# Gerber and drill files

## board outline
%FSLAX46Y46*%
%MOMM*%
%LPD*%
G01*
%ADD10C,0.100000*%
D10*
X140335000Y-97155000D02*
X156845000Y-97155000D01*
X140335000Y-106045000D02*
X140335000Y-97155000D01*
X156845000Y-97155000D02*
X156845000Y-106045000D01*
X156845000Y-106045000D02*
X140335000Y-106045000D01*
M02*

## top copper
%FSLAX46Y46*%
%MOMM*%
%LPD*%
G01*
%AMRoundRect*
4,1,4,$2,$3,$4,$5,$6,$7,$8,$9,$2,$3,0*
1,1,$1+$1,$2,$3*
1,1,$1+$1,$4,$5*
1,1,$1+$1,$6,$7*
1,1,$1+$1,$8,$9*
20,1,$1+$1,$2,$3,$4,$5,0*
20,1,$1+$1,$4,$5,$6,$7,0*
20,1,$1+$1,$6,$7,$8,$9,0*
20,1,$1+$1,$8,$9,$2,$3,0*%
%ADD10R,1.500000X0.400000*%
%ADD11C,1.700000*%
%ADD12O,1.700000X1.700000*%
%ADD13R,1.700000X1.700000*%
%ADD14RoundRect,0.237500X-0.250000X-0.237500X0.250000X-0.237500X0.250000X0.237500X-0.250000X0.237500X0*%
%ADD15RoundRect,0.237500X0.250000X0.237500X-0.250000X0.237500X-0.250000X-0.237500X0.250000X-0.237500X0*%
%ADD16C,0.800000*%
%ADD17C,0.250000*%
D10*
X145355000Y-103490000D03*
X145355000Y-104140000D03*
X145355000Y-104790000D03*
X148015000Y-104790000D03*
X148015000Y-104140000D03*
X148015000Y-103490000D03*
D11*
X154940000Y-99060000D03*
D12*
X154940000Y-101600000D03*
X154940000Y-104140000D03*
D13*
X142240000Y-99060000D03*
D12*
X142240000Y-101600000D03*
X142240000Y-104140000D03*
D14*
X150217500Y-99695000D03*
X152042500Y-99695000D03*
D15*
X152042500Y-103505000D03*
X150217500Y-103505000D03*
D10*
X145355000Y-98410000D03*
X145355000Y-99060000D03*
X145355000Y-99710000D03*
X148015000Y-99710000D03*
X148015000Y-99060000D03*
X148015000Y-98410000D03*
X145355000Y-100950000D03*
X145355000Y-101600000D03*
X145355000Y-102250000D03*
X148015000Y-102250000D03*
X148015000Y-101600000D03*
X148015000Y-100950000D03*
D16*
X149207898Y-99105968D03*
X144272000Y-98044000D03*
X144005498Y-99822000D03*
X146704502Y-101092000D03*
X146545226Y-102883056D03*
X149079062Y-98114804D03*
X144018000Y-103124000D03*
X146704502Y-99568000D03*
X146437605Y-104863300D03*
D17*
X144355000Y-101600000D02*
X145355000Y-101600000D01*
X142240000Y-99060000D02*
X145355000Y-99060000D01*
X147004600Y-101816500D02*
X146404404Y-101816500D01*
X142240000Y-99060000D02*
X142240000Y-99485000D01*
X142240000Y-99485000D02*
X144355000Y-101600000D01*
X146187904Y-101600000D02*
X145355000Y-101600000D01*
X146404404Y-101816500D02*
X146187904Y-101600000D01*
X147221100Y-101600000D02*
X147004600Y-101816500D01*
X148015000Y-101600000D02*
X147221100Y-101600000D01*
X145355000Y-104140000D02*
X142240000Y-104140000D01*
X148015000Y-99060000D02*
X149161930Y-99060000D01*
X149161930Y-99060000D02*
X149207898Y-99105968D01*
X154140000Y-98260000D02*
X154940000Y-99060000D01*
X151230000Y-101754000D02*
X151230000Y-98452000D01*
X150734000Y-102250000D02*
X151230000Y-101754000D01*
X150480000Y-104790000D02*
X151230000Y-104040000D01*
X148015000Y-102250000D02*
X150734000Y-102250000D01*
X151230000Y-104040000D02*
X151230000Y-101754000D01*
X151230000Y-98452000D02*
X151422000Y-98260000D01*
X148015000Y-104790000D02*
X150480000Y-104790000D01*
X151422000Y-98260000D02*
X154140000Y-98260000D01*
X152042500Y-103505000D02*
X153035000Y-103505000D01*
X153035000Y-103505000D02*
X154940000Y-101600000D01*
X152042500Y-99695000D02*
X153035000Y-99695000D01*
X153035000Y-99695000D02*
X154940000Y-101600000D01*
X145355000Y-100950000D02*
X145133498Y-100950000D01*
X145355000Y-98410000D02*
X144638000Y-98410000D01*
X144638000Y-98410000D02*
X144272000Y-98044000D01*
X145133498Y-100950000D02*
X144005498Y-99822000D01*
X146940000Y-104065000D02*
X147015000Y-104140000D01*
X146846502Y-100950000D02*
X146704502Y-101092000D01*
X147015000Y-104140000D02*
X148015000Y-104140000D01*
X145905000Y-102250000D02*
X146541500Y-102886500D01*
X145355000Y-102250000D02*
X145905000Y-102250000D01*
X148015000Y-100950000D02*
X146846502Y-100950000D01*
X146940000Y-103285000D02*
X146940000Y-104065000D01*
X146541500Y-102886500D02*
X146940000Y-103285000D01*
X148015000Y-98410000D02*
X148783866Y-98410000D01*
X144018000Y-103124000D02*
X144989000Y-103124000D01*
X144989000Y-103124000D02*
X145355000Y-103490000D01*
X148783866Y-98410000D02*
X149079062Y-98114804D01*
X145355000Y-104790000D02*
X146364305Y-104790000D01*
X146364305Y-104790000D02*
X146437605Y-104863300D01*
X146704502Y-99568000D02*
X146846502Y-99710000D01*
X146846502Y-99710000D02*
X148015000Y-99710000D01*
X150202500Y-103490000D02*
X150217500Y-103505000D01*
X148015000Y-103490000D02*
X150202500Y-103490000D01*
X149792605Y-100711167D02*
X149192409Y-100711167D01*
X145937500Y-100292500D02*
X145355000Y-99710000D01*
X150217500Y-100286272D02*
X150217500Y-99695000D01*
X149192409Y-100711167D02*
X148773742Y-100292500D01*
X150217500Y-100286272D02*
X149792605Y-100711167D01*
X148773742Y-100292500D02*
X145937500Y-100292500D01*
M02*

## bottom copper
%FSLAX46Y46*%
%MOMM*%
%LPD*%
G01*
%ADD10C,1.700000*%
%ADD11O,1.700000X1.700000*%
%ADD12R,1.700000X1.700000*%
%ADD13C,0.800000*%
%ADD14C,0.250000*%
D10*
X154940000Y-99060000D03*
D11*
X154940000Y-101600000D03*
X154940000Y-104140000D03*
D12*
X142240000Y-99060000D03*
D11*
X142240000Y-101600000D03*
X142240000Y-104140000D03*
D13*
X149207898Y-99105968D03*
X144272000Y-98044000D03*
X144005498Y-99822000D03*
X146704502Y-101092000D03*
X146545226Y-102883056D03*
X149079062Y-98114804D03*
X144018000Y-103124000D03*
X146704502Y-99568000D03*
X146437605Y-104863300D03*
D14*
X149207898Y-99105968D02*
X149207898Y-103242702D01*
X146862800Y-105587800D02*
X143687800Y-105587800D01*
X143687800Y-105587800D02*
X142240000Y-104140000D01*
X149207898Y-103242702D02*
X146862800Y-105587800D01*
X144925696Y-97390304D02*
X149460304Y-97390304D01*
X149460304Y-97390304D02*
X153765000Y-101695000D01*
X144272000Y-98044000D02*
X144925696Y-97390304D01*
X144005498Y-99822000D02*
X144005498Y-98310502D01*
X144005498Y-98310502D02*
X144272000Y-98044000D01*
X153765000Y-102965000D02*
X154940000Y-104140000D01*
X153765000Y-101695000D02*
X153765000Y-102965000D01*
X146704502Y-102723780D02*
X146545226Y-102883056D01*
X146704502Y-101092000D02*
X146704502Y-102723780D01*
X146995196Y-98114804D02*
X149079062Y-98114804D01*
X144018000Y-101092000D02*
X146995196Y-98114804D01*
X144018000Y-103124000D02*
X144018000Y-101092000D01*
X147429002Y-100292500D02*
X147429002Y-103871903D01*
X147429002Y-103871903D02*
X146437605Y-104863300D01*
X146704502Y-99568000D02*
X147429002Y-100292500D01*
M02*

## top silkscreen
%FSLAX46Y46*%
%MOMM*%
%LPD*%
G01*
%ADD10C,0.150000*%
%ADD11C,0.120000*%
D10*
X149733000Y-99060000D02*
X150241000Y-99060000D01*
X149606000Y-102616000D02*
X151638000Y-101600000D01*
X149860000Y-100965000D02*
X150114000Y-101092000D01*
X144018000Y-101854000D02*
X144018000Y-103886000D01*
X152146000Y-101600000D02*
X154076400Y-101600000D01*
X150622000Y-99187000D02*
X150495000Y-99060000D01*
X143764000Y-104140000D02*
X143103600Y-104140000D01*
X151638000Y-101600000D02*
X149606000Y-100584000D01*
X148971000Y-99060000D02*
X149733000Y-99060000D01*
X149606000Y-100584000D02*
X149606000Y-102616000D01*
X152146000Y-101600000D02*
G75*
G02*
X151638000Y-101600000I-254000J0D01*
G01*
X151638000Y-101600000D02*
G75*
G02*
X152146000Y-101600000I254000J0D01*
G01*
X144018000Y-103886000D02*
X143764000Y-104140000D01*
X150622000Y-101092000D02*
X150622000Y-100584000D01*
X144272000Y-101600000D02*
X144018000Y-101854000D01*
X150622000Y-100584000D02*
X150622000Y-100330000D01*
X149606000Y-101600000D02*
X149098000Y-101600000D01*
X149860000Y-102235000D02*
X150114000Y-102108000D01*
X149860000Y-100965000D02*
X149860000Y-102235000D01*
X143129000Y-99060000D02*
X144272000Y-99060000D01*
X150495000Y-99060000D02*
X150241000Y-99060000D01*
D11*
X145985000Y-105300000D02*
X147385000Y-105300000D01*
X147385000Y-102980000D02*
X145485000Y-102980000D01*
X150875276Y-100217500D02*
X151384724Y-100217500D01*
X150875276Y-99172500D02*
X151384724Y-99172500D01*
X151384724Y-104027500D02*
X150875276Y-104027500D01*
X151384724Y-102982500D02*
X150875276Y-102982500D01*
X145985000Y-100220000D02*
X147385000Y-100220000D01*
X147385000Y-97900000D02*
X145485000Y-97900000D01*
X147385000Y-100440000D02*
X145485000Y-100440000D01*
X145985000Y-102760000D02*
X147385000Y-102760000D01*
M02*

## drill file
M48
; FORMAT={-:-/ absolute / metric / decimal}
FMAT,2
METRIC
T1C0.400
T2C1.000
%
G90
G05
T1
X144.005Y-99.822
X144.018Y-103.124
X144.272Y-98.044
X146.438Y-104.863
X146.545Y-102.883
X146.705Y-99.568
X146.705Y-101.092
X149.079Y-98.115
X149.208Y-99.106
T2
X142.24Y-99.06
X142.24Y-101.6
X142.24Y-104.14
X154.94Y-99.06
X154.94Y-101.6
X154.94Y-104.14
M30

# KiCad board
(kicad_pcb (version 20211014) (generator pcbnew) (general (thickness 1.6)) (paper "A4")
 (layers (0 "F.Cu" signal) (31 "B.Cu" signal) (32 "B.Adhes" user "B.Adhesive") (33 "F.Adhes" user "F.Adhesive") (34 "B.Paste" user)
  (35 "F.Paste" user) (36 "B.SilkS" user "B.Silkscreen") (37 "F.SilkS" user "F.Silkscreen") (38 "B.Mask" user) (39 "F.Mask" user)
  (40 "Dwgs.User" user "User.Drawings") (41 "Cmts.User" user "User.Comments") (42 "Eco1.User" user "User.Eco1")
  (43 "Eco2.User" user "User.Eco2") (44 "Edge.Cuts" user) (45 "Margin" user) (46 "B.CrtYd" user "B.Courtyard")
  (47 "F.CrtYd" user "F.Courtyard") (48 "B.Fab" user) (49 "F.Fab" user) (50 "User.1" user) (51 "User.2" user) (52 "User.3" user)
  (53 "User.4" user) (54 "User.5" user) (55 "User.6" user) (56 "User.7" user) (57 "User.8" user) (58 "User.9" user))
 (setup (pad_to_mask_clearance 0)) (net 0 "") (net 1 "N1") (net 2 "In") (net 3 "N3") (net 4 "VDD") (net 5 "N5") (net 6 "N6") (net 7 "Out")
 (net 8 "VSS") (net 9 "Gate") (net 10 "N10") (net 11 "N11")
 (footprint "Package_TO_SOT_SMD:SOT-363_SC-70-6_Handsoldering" (layer "F.Cu") (at 146.685 104.14)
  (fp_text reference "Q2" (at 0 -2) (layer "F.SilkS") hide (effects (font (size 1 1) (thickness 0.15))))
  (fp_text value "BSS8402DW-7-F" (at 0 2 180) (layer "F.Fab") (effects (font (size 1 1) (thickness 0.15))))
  (fp_line (start -0.7 1.16) (end 0.7 1.16) (layer "F.SilkS") (width 0.12))
  (fp_line (start 0.7 -1.16) (end -1.2 -1.16) (layer "F.SilkS") (width 0.12))
  (pad "1" smd rect (at -1.33 -0.65) (size 1.5 0.4) (layers "F.Cu" "F.Paste" "F.Mask") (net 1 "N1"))
  (pad "2" smd rect (at -1.33 0) (size 1.5 0.4) (layers "F.Cu" "F.Paste" "F.Mask") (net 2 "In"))
  (pad "3" smd rect (at -1.33 0.65) (size 1.5 0.4) (layers "F.Cu" "F.Paste" "F.Mask") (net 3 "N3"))
  (pad "4" smd rect (at 1.33 0.65) (size 1.5 0.4) (layers "F.Cu" "F.Paste" "F.Mask") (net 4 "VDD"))
  (pad "5" smd rect (at 1.33 0) (size 1.5 0.4) (layers "F.Cu" "F.Paste" "F.Mask") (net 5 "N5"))
  (pad "6" smd rect (at 1.33 -0.65) (size 1.5 0.4) (layers "F.Cu" "F.Paste" "F.Mask") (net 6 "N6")))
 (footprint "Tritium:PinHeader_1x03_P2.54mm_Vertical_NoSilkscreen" (layer "F.Cu") (at 154.94 99.06)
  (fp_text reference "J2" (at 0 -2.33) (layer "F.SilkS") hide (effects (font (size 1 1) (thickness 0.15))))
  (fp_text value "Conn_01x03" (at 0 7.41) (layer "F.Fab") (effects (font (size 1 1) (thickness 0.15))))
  (pad "1" thru_hole circle (at 0 0) (size 1.7 1.7) (drill 1) (layers *.Cu *.Mask) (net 4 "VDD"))
  (pad "2" thru_hole oval (at 0 2.54) (size 1.7 1.7) (drill 1) (layers *.Cu *.Mask) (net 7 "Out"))
  (pad "3" thru_hole oval (at 0 5.08) (size 1.7 1.7) (drill 1) (layers *.Cu *.Mask) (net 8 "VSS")))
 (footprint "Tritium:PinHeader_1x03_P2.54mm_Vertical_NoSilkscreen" (layer "F.Cu") (at 142.24 99.06)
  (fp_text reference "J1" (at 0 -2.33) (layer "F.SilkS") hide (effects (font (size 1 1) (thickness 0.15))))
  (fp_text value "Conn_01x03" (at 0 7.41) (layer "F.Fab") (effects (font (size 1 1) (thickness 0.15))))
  (pad "1" thru_hole rect (at 0 0) (size 1.7 1.7) (drill 1) (layers *.Cu *.Mask) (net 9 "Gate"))
  (pad "2" thru_hole oval (at 0 2.54) (size 1.7 1.7) (drill 1) (layers *.Cu *.Mask) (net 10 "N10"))
  (pad "3" thru_hole oval (at 0 5.08) (size 1.7 1.7) (drill 1) (layers *.Cu *.Mask) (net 2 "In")))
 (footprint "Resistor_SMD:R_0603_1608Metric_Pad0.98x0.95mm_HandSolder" (layer "F.Cu") (at 151.13 99.695)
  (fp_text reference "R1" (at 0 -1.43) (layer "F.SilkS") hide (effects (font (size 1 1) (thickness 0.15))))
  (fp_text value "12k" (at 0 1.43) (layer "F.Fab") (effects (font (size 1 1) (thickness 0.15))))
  (fp_line (start -0.254724 0.5225) (end 0.254724 0.5225) (layer "F.SilkS") (width 0.12))
  (fp_line (start -0.254724 -0.5225) (end 0.254724 -0.5225) (layer "F.SilkS") (width 0.12))
  (pad "1" smd roundrect (at -0.9125 0) (size 0.975 0.95) (layers "F.Cu" "F.Paste" "F.Mask") (roundrect_rratio 0.25) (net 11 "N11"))
  (pad "2" smd roundrect (at 0.9125 0) (size 0.975 0.95) (layers "F.Cu" "F.Paste" "F.Mask") (roundrect_rratio 0.25) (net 7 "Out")))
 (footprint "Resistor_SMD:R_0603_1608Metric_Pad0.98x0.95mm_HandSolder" (layer "F.Cu") (at 151.13 103.505 180)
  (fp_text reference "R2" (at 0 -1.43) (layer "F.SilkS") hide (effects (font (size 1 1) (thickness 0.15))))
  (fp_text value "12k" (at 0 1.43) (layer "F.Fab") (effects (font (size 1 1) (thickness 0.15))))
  (fp_line (start -0.254724 -0.5225) (end 0.254724 -0.5225) (layer "F.SilkS") (width 0.12))
  (fp_line (start -0.254724 0.5225) (end 0.254724 0.5225) (layer "F.SilkS") (width 0.12))
  (pad "1" smd roundrect (at -0.9125 0 180) (size 0.975 0.95) (layers "F.Cu" "F.Paste" "F.Mask") (roundrect_rratio 0.25) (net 7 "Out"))
  (pad "2" smd roundrect (at 0.9125 0 180) (size 0.975 0.95) (layers "F.Cu" "F.Paste" "F.Mask") (roundrect_rratio 0.25) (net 6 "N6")))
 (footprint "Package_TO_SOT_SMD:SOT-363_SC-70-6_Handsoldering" (layer "F.Cu") (at 146.685 99.06)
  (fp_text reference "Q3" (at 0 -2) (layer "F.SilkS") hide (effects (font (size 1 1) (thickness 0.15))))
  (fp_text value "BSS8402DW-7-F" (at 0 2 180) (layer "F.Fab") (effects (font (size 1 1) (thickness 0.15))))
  (fp_line (start -0.7 1.16) (end 0.7 1.16) (layer "F.SilkS") (width 0.12))
  (fp_line (start 0.7 -1.16) (end -1.2 -1.16) (layer "F.SilkS") (width 0.12))
  (pad "1" smd rect (at -1.33 -0.65) (size 1.5 0.4) (layers "F.Cu" "F.Paste" "F.Mask") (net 8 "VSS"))
  (pad "2" smd rect (at -1.33 0) (size 1.5 0.4) (layers "F.Cu" "F.Paste" "F.Mask") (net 9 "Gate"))
  (pad "3" smd rect (at -1.33 0.65) (size 1.5 0.4) (layers "F.Cu" "F.Paste" "F.Mask") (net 11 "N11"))
  (pad "4" smd rect (at 1.33 0.65) (size 1.5 0.4) (layers "F.Cu" "F.Paste" "F.Mask") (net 3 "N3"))
  (pad "5" smd rect (at 1.33 0) (size 1.5 0.4) (layers "F.Cu" "F.Paste" "F.Mask") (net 2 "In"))
  (pad "6" smd rect (at 1.33 -0.65) (size 1.5 0.4) (layers "F.Cu" "F.Paste" "F.Mask") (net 1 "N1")))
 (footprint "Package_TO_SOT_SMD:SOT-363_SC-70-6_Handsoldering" (layer "F.Cu") (at 146.685 101.6)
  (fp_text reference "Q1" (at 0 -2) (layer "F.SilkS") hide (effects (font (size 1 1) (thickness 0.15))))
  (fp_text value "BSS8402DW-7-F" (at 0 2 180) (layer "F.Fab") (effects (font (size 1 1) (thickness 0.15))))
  (fp_line (start 0.7 -1.16) (end -1.2 -1.16) (layer "F.SilkS") (width 0.12))
  (fp_line (start -0.7 1.16) (end 0.7 1.16) (layer "F.SilkS") (width 0.12))
  (pad "1" smd rect (at -1.33 -0.65) (size 1.5 0.4) (layers "F.Cu" "F.Paste" "F.Mask") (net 8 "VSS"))
  (pad "2" smd rect (at -1.33 0) (size 1.5 0.4) (layers "F.Cu" "F.Paste" "F.Mask") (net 9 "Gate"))
  (pad "3" smd rect (at -1.33 0.65) (size 1.5 0.4) (layers "F.Cu" "F.Paste" "F.Mask") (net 5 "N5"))
  (pad "4" smd rect (at 1.33 0.65) (size 1.5 0.4) (layers "F.Cu" "F.Paste" "F.Mask") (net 4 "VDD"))
  (pad "5" smd rect (at 1.33 0) (size 1.5 0.4) (layers "F.Cu" "F.Paste" "F.Mask") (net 9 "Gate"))
  (pad "6" smd rect (at 1.33 -0.65) (size 1.5 0.4) (layers "F.Cu" "F.Paste" "F.Mask") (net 5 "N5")))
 (gr_line (start 149.733 99.06) (end 150.241 99.06) (layer "F.SilkS") (width 0.15))
 (gr_line (start 149.606 102.616) (end 151.638 101.6) (layer "F.SilkS") (width 0.15))
 (gr_line (start 149.86 100.965) (end 150.114 101.092) (layer "F.SilkS") (width 0.15))
 (gr_line (start 144.018 101.854) (end 144.018 103.886) (layer "F.SilkS") (width 0.15))
 (gr_line (start 152.146 101.6) (end 154.0764 101.6) (layer "F.SilkS") (width 0.15))
 (gr_line (start 150.622 99.187) (end 150.495 99.06) (layer "F.SilkS") (width 0.15))
 (gr_line (start 143.764 104.14) (end 143.1036 104.14) (layer "F.SilkS") (width 0.15))
 (gr_line (start 151.638 101.6) (end 149.606 100.584) (layer "F.SilkS") (width 0.15))
 (gr_line (start 148.971 99.06) (end 149.733 99.06) (layer "F.SilkS") (width 0.15))
 (gr_line (start 149.606 100.584) (end 149.606 102.616) (layer "F.SilkS") (width 0.15))
 (gr_circle (center 151.892 101.6) (end 152.146 101.6) (layer "F.SilkS") (width 0.15) (fill none))
 (gr_line (start 144.018 103.886) (end 143.764 104.14) (layer "F.SilkS") (width 0.15))
 (gr_line (start 150.622 101.092) (end 150.622 100.584) (layer "F.SilkS") (width 0.15))
 (gr_line (start 144.272 101.6) (end 144.018 101.854) (layer "F.SilkS") (width 0.15))
 (gr_line (start 150.622 100.584) (end 150.622 100.33) (layer "F.SilkS") (width 0.15))
 (gr_line (start 149.606 101.6) (end 149.098 101.6) (layer "F.SilkS") (width 0.15))
 (gr_line (start 149.86 102.235) (end 150.114 102.108) (layer "F.SilkS") (width 0.15))
 (gr_line (start 149.86 100.965) (end 149.86 102.235) (layer "F.SilkS") (width 0.15))
 (gr_line (start 143.129 99.06) (end 144.272 99.06) (layer "F.SilkS") (width 0.15))
 (gr_line (start 150.495 99.06) (end 150.241 99.06) (layer "F.SilkS") (width 0.15))
 (gr_line (start 140.335 97.155) (end 156.845 97.155) (layer "Edge.Cuts") (width 0.1))
 (gr_line (start 140.335 106.045) (end 140.335 97.155) (layer "Edge.Cuts") (width 0.1))
 (gr_line (start 156.845 97.155) (end 156.845 106.045) (layer "Edge.Cuts") (width 0.1))
 (gr_line (start 156.845 106.045) (end 140.335 106.045) (layer "Edge.Cuts") (width 0.1))
 (segment (start 144.355 101.6) (end 145.355 101.6) (width 0.25) (layer "F.Cu") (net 9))
 (segment (start 142.24 99.06) (end 145.355 99.06) (width 0.25) (layer "F.Cu") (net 9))
 (segment (start 147.0046 101.8165) (end 146.404404 101.8165) (width 0.25) (layer "F.Cu") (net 9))
 (segment (start 142.24 99.06) (end 142.24 99.485) (width 0.25) (layer "F.Cu") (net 9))
 (segment (start 142.24 99.485) (end 144.355 101.6) (width 0.25) (layer "F.Cu") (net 9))
 (segment (start 146.187904 101.6) (end 145.355 101.6) (width 0.25) (layer "F.Cu") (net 9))
 (segment (start 146.404404 101.8165) (end 146.187904 101.6) (width 0.25) (layer "F.Cu") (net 9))
 (segment (start 147.2211 101.6) (end 147.0046 101.8165) (width 0.25) (layer "F.Cu") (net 9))
 (segment (start 148.015 101.6) (end 147.2211 101.6) (width 0.25) (layer "F.Cu") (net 9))
 (segment (start 145.355 104.14) (end 142.24 104.14) (width 0.25) (layer "F.Cu") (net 2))
 (segment (start 148.015 99.06) (end 149.16193 99.06) (width 0.25) (layer "F.Cu") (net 2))
 (segment (start 149.16193 99.06) (end 149.207898 99.105968) (width 0.25) (layer "F.Cu") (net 2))
 (via (at 149.207898 99.105968) (size 0.8) (drill 0.4) (layers "F.Cu" "B.Cu") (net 2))
 (segment (start 149.207898 99.105968) (end 149.207898 103.242702) (width 0.25) (layer "B.Cu") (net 2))
 (segment (start 146.8628 105.5878) (end 143.6878 105.5878) (width 0.25) (layer "B.Cu") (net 2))
 (segment (start 143.6878 105.5878) (end 142.24 104.14) (width 0.25) (layer "B.Cu") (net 2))
 (segment (start 149.207898 103.242702) (end 146.8628 105.5878) (width 0.25) (layer "B.Cu") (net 2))
 (segment (start 154.14 98.26) (end 154.94 99.06) (width 0.25) (layer "F.Cu") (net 4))
 (segment (start 151.23 101.754) (end 151.23 98.452) (width 0.25) (layer "F.Cu") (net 4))
 (segment (start 150.734 102.25) (end 151.23 101.754) (width 0.25) (layer "F.Cu") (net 4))
 (segment (start 150.48 104.79) (end 151.23 104.04) (width 0.25) (layer "F.Cu") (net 4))
 (segment (start 148.015 102.25) (end 150.734 102.25) (width 0.25) (layer "F.Cu") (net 4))
 (segment (start 151.23 104.04) (end 151.23 101.754) (width 0.25) (layer "F.Cu") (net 4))
 (segment (start 151.23 98.452) (end 151.422 98.26) (width 0.25) (layer "F.Cu") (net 4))
 (segment (start 148.015 104.79) (end 150.48 104.79) (width 0.25) (layer "F.Cu") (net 4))
 (segment (start 151.422 98.26) (end 154.14 98.26) (width 0.25) (layer "F.Cu") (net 4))
 (segment (start 152.0425 103.505) (end 153.035 103.505) (width 0.25) (layer "F.Cu") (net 7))
 (segment (start 153.035 103.505) (end 154.94 101.6) (width 0.25) (layer "F.Cu") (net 7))
 (segment (start 152.0425 99.695) (end 153.035 99.695) (width 0.25) (layer "F.Cu") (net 7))
 (segment (start 153.035 99.695) (end 154.94 101.6) (width 0.25) (layer "F.Cu") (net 7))
 (segment (start 145.355 100.95) (end 145.133498 100.95) (width 0.25) (layer "F.Cu") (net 8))
 (segment (start 145.355 98.41) (end 144.638 98.41) (width 0.25) (layer "F.Cu") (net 8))
 (segment (start 144.638 98.41) (end 144.272 98.044) (width 0.25) (layer "F.Cu") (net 8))
 (segment (start 145.133498 100.95) (end 144.005498 99.822) (width 0.25) (layer "F.Cu") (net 8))
 (via (at 144.272 98.044) (size 0.8) (drill 0.4) (layers "F.Cu" "B.Cu") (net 8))
 (via (at 144.005498 99.822) (size 0.8) (drill 0.4) (layers "F.Cu" "B.Cu") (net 8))
 (segment (start 144.925696 97.390304) (end 149.460304 97.390304) (width 0.25) (layer "B.Cu") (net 8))
 (segment (start 149.460304 97.390304) (end 153.765 101.695) (width 0.25) (layer "B.Cu") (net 8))
 (segment (start 144.272 98.044) (end 144.925696 97.390304) (width 0.25) (layer "B.Cu") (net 8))
 (segment (start 144.005498 99.822) (end 144.005498 98.310502) (width 0.25) (layer "B.Cu") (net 8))
 (segment (start 144.005498 98.310502) (end 144.272 98.044) (width 0.25) (layer "B.Cu") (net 8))
 (segment (start 153.765 102.965) (end 154.94 104.14) (width 0.25) (layer "B.Cu") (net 8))
 (segment (start 153.765 101.695) (end 153.765 102.965) (width 0.25) (layer "B.Cu") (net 8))
 (segment (start 146.94 104.065) (end 147.015 104.14) (width 0.25) (layer "F.Cu") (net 5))
 (segment (start 146.846502 100.95) (end 146.704502 101.092) (width 0.25) (layer "F.Cu") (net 5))
 (segment (start 147.015 104.14) (end 148.015 104.14) (width 0.25) (layer "F.Cu") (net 5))
 (segment (start 145.905 102.25) (end 146.5415 102.8865) (width 0.25) (layer "F.Cu") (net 5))
 (segment (start 145.355 102.25) (end 145.905 102.25) (width 0.25) (layer "F.Cu") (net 5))
 (segment (start 148.015 100.95) (end 146.846502 100.95) (width 0.25) (layer "F.Cu") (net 5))
 (segment (start 146.94 103.285) (end 146.94 104.065) (width 0.25) (layer "F.Cu") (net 5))
 (segment (start 146.5415 102.8865) (end 146.94 103.285) (width 0.25) (layer "F.Cu") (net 5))
 (via (at 146.704502 101.092) (size 0.8) (drill 0.4) (layers "F.Cu" "B.Cu") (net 5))
 (via (at 146.545226 102.883056) (size 0.8) (drill 0.4) (layers "F.Cu" "B.Cu") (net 5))
 (segment (start 146.704502 102.72378) (end 146.545226 102.883056) (width 0.25) (layer "B.Cu") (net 5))
 (segment (start 146.704502 101.092) (end 146.704502 102.72378) (width 0.25) (layer "B.Cu") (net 5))
 (segment (start 148.015 98.41) (end 148.783866 98.41) (width 0.25) (layer "F.Cu") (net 1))
 (segment (start 144.018 103.124) (end 144.989 103.124) (width 0.25) (layer "F.Cu") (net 1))
 (segment (start 144.989 103.124) (end 145.355 103.49) (width 0.25) (layer "F.Cu") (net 1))
 (segment (start 148.783866 98.41) (end 149.079062 98.114804) (width 0.25) (layer "F.Cu") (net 1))
 (via (at 149.079062 98.114804) (size 0.8) (drill 0.4) (layers "F.Cu" "B.Cu") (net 1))
 (via (at 144.018 103.124) (size 0.8) (drill 0.4) (layers "F.Cu" "B.Cu") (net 1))
 (segment (start 146.995196 98.114804) (end 149.079062 98.114804) (width 0.25) (layer "B.Cu") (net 1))
 (segment (start 144.018 101.092) (end 146.995196 98.114804) (width 0.25) (layer "B.Cu") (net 1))
 (segment (start 144.018 103.124) (end 144.018 101.092) (width 0.25) (layer "B.Cu") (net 1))
 (segment (start 145.355 104.79) (end 146.364305 104.79) (width 0.25) (layer "F.Cu") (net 3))
 (segment (start 146.364305 104.79) (end 146.437605 104.8633) (width 0.25) (layer "F.Cu") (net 3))
 (segment (start 146.704502 99.568) (end 146.846502 99.71) (width 0.25) (layer "F.Cu") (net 3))
 (segment (start 146.846502 99.71) (end 148.015 99.71) (width 0.25) (layer "F.Cu") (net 3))
 (via (at 146.704502 99.568) (size 0.8) (drill 0.4) (layers "F.Cu" "B.Cu") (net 3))
 (via (at 146.437605 104.8633) (size 0.8) (drill 0.4) (layers "F.Cu" "B.Cu") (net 3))
 (segment (start 147.429002 100.2925) (end 147.429002 103.871903) (width 0.25) (layer "B.Cu") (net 3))
 (segment (start 147.429002 103.871903) (end 146.437605 104.8633) (width 0.25) (layer "B.Cu") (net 3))
 (segment (start 146.704502 99.568) (end 147.429002 100.2925) (width 0.25) (layer "B.Cu") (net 3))
 (segment (start 150.2025 103.49) (end 150.2175 103.505) (width 0.25) (layer "F.Cu") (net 6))
 (segment (start 148.015 103.49) (end 150.2025 103.49) (width 0.25) (layer "F.Cu") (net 6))
 (segment (start 149.792605 100.711167) (end 149.192409 100.711167) (width 0.25) (layer "F.Cu") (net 11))
 (segment (start 145.9375 100.2925) (end 145.355 99.71) (width 0.25) (layer "F.Cu") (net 11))
 (segment (start 150.2175 100.286272) (end 150.2175 99.695) (width 0.25) (layer "F.Cu") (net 11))
 (segment (start 149.192409 100.711167) (end 148.773742 100.2925) (width 0.25) (layer "F.Cu") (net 11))
 (segment (start 150.2175 100.286272) (end 149.792605 100.711167) (width 0.25) (layer "F.Cu") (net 11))
 (segment (start 148.773742 100.2925) (end 145.9375 100.2925) (width 0.25) (layer "F.Cu") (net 11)))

